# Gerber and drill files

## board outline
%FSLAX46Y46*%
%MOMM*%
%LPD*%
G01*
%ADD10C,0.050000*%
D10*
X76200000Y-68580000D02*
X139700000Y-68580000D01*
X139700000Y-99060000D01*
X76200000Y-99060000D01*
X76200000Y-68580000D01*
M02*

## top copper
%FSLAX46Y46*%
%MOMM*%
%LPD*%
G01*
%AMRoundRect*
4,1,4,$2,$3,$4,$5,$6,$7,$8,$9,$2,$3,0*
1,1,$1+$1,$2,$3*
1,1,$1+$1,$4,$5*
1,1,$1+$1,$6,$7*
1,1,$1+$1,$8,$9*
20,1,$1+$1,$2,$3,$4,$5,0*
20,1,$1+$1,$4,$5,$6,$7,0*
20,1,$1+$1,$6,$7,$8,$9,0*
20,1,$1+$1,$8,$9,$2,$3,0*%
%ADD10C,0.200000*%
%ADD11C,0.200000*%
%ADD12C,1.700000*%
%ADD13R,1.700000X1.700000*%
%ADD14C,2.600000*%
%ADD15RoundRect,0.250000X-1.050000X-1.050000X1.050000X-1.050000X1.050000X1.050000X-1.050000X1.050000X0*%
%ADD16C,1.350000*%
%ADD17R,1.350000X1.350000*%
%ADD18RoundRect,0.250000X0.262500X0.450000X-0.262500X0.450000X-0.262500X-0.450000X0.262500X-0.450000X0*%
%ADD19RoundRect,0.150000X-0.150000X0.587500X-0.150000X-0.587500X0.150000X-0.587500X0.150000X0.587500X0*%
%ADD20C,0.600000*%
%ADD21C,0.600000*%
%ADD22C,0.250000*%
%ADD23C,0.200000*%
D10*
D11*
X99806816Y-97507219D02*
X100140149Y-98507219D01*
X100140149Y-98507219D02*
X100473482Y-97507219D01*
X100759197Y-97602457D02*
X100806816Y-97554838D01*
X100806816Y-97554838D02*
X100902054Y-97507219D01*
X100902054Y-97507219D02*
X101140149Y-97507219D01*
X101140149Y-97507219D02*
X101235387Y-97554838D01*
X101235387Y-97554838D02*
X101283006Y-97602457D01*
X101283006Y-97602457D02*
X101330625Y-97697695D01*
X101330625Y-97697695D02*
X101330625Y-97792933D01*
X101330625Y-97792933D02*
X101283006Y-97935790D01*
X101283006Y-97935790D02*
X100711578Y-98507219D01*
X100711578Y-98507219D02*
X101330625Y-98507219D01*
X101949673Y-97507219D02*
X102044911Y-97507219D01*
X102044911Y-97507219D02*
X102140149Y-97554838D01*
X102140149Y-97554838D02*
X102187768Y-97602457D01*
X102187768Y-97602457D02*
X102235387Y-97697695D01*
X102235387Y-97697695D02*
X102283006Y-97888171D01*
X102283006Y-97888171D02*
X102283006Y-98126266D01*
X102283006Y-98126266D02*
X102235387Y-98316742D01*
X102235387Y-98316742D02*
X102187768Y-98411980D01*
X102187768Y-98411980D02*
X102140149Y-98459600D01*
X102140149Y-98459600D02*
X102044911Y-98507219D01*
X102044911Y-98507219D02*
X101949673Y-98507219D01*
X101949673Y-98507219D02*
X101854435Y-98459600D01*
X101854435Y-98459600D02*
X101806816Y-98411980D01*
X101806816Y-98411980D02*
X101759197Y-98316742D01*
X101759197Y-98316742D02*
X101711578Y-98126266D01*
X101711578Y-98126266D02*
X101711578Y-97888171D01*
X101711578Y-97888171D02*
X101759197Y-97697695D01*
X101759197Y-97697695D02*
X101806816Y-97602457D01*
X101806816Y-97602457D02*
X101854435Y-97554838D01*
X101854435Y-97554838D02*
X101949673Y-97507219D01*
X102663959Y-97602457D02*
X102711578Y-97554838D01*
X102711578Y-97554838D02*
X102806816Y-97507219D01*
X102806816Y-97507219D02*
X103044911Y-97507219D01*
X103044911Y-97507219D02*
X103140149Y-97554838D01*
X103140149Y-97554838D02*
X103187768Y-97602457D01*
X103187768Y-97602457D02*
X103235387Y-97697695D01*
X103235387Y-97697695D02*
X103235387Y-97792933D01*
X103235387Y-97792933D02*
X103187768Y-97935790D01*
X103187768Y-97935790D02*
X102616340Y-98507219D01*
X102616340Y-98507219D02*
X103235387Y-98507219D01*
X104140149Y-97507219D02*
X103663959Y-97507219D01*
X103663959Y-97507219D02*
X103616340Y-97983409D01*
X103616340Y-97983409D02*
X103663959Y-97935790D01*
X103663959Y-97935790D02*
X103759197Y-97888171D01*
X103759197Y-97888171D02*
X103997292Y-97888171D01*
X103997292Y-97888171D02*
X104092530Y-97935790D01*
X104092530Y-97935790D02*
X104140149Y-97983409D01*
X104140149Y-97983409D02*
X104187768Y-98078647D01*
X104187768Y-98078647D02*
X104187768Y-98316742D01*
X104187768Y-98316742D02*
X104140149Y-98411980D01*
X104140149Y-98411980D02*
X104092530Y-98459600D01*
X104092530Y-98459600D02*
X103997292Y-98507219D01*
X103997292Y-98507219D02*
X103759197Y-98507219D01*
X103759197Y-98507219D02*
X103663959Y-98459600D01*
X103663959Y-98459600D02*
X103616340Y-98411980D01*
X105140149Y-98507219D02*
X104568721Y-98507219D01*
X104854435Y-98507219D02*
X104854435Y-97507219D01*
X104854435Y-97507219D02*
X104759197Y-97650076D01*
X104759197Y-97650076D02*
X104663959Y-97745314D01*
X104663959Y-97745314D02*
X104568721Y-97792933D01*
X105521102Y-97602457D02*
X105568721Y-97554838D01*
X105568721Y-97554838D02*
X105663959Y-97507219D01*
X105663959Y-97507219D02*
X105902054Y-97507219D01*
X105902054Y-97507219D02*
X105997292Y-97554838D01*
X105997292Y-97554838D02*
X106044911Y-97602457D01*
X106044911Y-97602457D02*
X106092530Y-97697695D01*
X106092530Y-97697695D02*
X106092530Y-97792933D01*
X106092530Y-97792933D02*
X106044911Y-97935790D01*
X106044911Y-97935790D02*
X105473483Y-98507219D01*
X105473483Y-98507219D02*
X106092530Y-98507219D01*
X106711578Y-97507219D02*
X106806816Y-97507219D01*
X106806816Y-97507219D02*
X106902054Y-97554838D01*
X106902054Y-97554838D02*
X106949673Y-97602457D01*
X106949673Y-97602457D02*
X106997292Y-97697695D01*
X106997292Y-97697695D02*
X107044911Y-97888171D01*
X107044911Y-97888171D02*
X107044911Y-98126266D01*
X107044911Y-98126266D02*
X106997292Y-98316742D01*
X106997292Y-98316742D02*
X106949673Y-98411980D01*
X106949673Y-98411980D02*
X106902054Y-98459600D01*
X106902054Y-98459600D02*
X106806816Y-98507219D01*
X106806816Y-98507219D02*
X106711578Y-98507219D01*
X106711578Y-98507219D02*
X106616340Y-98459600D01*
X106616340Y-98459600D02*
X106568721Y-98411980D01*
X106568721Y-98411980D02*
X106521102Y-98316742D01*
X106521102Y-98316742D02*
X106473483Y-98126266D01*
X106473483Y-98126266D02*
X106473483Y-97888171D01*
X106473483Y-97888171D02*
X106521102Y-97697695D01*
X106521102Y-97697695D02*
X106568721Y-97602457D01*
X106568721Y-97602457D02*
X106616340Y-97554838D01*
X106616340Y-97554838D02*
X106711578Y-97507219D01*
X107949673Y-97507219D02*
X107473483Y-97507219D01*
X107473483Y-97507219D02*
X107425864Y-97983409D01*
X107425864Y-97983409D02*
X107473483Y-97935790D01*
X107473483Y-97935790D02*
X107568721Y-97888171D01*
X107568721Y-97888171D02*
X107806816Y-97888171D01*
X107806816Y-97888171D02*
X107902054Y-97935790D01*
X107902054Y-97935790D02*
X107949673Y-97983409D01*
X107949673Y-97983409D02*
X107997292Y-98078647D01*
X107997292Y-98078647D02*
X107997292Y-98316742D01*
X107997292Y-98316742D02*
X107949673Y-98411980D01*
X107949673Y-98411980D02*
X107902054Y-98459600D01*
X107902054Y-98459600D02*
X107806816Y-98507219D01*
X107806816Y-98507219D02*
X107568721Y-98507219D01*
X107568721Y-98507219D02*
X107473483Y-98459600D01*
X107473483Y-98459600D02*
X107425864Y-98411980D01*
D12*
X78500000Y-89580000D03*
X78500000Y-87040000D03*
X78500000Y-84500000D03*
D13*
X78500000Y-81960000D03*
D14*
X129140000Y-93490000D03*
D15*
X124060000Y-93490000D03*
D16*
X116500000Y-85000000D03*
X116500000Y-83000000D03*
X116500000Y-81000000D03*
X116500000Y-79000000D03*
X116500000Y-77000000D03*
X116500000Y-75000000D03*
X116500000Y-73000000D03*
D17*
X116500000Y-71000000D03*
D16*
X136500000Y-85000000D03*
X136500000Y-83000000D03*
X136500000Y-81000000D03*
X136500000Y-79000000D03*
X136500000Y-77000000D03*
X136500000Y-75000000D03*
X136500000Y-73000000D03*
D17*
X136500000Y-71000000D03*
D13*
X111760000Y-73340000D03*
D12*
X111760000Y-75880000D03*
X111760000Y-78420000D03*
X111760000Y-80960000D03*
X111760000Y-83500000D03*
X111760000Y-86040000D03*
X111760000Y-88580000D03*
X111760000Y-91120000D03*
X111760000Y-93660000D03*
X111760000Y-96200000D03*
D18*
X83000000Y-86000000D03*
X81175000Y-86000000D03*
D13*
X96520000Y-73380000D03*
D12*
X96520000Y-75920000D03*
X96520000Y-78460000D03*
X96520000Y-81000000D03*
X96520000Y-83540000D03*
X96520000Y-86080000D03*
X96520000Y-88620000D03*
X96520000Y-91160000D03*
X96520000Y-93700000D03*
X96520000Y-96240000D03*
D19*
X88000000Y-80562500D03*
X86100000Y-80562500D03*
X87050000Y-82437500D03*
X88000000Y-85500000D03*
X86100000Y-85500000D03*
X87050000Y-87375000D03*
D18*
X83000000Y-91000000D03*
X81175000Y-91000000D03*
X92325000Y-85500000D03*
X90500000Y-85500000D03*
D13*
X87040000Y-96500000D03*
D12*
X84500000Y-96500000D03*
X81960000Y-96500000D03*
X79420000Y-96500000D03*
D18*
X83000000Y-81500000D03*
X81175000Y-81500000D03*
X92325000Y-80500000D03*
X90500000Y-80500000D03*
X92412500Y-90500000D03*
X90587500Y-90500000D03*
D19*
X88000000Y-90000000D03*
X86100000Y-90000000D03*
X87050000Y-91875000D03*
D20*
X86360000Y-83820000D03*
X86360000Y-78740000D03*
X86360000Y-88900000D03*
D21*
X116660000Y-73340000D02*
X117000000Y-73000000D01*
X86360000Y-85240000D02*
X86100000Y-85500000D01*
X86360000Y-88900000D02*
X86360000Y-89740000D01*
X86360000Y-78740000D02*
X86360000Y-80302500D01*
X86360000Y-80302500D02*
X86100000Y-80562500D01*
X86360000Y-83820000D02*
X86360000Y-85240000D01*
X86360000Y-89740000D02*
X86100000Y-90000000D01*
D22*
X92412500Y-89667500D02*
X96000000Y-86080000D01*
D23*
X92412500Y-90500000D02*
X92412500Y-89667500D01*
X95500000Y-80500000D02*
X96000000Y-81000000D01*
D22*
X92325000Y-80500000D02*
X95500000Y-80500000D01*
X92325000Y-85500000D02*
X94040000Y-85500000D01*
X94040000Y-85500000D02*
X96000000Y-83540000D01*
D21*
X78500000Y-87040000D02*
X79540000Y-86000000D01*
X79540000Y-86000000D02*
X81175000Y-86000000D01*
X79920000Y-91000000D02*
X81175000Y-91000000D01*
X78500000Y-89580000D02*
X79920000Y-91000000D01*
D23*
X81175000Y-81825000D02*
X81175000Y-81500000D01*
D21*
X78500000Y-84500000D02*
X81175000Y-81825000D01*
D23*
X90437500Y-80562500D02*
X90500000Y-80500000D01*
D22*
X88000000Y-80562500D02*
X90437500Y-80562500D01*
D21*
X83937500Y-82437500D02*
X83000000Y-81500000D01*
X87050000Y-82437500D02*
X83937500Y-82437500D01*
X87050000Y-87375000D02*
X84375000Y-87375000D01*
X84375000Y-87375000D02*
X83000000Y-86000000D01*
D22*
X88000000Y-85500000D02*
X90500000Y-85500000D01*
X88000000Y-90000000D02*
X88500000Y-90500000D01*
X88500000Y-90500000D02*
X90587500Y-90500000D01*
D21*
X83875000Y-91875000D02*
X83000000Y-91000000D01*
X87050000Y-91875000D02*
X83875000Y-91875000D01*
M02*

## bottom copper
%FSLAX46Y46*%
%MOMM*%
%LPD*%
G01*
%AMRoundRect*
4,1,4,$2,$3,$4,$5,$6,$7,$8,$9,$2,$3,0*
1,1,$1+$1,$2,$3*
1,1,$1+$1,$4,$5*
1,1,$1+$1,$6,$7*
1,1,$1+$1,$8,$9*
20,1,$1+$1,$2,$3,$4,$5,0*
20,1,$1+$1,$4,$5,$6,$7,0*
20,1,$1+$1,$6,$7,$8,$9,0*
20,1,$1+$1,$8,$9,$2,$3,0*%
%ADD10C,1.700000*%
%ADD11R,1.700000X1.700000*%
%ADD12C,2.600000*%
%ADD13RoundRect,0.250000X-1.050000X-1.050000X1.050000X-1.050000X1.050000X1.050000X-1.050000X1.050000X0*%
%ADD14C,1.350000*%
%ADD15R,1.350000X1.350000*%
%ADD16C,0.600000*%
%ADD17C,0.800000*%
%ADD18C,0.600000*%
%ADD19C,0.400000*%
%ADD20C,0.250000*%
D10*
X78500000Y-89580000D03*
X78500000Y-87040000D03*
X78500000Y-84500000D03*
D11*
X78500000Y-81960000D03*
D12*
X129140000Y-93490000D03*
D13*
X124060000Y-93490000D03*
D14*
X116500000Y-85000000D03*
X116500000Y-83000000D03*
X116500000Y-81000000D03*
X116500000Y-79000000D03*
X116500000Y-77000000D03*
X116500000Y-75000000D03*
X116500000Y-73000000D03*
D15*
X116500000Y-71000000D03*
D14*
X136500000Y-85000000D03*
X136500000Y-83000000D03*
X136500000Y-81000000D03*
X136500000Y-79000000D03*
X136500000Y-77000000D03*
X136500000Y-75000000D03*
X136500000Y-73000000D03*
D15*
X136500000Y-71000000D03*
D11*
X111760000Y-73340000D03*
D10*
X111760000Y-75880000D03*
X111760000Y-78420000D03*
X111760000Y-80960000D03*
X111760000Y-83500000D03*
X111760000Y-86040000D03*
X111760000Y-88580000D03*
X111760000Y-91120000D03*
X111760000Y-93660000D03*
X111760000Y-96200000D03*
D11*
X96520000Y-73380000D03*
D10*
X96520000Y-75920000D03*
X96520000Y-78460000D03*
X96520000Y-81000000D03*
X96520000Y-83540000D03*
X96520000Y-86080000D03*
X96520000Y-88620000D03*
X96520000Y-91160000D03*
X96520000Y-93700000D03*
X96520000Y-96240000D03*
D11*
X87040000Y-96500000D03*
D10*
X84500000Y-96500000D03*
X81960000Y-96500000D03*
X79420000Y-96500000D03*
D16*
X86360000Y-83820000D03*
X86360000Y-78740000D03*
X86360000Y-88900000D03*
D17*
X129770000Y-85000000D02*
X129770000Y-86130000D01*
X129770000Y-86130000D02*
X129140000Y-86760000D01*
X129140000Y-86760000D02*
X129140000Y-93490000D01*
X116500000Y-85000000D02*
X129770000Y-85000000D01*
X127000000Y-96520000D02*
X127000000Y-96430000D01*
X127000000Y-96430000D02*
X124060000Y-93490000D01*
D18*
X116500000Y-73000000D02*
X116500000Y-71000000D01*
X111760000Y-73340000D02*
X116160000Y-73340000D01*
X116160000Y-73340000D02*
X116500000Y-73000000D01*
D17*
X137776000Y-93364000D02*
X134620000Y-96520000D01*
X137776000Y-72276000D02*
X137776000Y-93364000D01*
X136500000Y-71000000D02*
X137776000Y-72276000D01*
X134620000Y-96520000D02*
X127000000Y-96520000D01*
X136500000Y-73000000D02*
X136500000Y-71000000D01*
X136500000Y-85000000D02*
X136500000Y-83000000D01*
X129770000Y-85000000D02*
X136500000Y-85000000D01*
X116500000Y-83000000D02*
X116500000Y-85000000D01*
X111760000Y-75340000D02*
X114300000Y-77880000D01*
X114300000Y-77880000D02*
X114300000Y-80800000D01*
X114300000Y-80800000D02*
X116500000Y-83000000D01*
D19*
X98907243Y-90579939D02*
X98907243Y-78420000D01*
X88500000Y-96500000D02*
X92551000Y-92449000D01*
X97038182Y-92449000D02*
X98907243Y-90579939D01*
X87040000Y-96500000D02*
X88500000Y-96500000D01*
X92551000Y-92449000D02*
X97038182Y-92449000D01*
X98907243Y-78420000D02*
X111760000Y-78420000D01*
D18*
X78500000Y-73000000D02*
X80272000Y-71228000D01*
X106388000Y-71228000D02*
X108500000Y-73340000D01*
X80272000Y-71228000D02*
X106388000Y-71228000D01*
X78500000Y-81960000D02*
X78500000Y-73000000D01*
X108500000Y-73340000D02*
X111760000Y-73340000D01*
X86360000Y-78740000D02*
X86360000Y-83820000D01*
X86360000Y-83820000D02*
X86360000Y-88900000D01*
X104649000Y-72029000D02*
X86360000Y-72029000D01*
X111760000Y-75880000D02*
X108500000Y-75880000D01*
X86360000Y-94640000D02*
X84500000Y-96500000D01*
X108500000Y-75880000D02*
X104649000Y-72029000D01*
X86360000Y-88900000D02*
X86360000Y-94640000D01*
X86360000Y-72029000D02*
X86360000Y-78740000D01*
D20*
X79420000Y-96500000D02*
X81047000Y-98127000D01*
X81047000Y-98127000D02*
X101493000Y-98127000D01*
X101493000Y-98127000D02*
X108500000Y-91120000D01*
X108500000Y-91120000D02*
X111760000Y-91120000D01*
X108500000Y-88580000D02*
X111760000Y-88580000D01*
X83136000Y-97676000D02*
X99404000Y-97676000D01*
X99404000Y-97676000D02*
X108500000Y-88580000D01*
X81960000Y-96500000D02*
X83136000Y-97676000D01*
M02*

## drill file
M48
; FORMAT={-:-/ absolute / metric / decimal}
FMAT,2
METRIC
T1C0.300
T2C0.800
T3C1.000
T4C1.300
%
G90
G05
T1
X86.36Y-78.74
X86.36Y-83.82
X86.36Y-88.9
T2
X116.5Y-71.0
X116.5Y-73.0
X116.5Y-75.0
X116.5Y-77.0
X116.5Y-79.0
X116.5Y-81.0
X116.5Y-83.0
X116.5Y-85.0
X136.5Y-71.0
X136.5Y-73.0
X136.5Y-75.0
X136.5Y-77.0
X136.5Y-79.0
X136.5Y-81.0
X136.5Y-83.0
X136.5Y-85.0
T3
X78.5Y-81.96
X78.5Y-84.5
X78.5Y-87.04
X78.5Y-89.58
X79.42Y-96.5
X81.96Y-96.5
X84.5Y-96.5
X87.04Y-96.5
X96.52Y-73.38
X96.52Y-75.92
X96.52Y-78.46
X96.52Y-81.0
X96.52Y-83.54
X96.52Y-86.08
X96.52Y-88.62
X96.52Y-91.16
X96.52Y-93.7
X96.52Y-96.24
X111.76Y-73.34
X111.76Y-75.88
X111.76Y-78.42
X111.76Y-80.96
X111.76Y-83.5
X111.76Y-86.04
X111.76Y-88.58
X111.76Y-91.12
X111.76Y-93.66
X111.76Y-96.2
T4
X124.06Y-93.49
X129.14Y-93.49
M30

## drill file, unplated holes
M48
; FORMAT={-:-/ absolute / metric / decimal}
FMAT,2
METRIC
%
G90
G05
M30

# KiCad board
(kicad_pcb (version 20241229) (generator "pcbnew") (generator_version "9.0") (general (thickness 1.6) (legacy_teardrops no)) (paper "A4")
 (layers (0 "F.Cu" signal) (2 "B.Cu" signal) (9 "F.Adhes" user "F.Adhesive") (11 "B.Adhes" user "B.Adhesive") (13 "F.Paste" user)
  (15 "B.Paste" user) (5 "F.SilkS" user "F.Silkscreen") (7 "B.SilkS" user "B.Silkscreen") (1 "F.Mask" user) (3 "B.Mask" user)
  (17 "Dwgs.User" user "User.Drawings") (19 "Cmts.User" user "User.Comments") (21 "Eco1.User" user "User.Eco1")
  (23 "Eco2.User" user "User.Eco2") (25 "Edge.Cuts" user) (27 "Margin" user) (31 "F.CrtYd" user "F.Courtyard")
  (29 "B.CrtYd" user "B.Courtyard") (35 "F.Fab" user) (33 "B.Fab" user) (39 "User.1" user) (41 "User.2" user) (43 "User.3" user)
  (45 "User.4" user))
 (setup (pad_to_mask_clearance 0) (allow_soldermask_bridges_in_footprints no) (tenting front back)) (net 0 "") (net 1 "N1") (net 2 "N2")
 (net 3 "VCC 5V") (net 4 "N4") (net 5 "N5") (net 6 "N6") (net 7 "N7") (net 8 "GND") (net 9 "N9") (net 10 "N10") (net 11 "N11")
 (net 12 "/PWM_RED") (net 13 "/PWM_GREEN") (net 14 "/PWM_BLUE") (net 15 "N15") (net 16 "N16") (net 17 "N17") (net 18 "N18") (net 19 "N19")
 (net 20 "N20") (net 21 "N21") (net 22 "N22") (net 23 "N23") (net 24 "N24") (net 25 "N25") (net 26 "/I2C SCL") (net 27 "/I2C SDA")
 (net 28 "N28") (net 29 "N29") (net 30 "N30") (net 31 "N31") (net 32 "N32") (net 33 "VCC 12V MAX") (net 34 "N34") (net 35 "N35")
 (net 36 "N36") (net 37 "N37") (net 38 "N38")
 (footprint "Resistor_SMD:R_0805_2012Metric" (layer "F.Cu") (at 82.0875 86 180)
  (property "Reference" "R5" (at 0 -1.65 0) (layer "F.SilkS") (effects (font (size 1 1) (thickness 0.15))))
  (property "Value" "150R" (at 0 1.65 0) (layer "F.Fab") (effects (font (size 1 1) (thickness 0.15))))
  (pad "1" smd roundrect (at -0.9125 0 180) (size 1.025 1.4) (layers "F.Cu" "F.Mask" "F.Paste") (roundrect_rratio 0.243902) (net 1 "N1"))
  (pad "2" smd roundrect (at 0.9125 0 180) (size 1.025 1.4) (layers "F.Cu" "F.Mask" "F.Paste") (roundrect_rratio 0.243902) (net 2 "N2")))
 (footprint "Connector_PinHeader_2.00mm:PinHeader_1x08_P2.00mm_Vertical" (layer "F.Cu") (at 116.5 71)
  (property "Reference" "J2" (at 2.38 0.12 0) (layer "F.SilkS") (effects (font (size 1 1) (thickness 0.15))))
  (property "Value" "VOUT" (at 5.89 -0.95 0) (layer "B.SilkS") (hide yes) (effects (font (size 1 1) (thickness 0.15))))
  (pad "1" thru_hole rect (at 0 0) (size 1.35 1.35) (drill 0.8) (layers "*.Cu" "*.Mask") (remove_unused_layers no) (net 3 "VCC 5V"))
  (pad "2" thru_hole circle (at 0 2) (size 1.35 1.35) (drill 0.8) (layers "*.Cu" "*.Mask") (remove_unused_layers no) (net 3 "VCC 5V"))
  (pad "3" thru_hole circle (at 0 4) (size 1.35 1.35) (drill 0.8) (layers "*.Cu" "*.Mask") (remove_unused_layers no) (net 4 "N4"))
  (pad "4" thru_hole circle (at 0 6) (size 1.35 1.35) (drill 0.8) (layers "*.Cu" "*.Mask") (remove_unused_layers no) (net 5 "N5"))
  (pad "5" thru_hole circle (at 0 8) (size 1.35 1.35) (drill 0.8) (layers "*.Cu" "*.Mask") (remove_unused_layers no) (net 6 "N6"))
  (pad "6" thru_hole circle (at 0 10) (size 1.35 1.35) (drill 0.8) (layers "*.Cu" "*.Mask") (remove_unused_layers no) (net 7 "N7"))
  (pad "7" thru_hole circle (at 0 12) (size 1.35 1.35) (drill 0.8) (layers "*.Cu" "*.Mask") (remove_unused_layers no) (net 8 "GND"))
  (pad "8" thru_hole circle (at 0 14) (size 1.35 1.35) (drill 0.8) (layers "*.Cu" "*.Mask") (remove_unused_layers no) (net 8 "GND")))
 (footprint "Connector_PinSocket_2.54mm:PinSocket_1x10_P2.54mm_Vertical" (layer "F.Cu") (at 96.52 73.38)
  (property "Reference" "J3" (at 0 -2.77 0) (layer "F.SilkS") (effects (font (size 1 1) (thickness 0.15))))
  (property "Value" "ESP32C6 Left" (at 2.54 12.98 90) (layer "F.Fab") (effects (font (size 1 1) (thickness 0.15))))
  (pad "1" thru_hole rect (at 0 0) (size 1.7 1.7) (drill 1) (layers "*.Cu" "*.Mask") (remove_unused_layers no) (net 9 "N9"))
  (pad "2" thru_hole circle (at 0 2.54) (size 1.7 1.7) (drill 1) (layers "*.Cu" "*.Mask") (remove_unused_layers no) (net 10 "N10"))
  (pad "3" thru_hole circle (at 0 5.08) (size 1.7 1.7) (drill 1) (layers "*.Cu" "*.Mask") (remove_unused_layers no) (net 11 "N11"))
  (pad "4" thru_hole circle (at 0 7.62) (size 1.7 1.7) (drill 1) (layers "*.Cu" "*.Mask") (remove_unused_layers no) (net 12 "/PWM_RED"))
  (pad "5" thru_hole circle (at 0 10.16) (size 1.7 1.7) (drill 1) (layers "*.Cu" "*.Mask") (remove_unused_layers no) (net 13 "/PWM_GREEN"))
  (pad "6" thru_hole circle (at 0 12.7) (size 1.7 1.7) (drill 1) (layers "*.Cu" "*.Mask") (remove_unused_layers no) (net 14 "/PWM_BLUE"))
  (pad "7" thru_hole circle (at 0 15.24) (size 1.7 1.7) (drill 1) (layers "*.Cu" "*.Mask") (remove_unused_layers no) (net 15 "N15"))
  (pad "8" thru_hole circle (at 0 17.78) (size 1.7 1.7) (drill 1) (layers "*.Cu" "*.Mask") (remove_unused_layers no) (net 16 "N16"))
  (pad "9" thru_hole circle (at 0 20.32) (size 1.7 1.7) (drill 1) (layers "*.Cu" "*.Mask") (remove_unused_layers no) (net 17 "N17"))
  (pad "10" thru_hole circle (at 0 22.86) (size 1.7 1.7) (drill 1) (layers "*.Cu" "*.Mask") (remove_unused_layers no) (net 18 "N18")))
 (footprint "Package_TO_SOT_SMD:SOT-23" (layer "F.Cu") (at 87.05 81.5 -90)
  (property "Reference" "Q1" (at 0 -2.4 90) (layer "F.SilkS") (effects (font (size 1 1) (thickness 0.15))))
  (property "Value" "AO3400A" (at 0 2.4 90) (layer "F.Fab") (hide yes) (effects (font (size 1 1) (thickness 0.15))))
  (pad "1" smd roundrect (at -0.9375 -0.95 270) (size 1.475 0.6) (layers "F.Cu" "F.Mask" "F.Paste") (roundrect_rratio 0.25) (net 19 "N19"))
  (pad "2" smd roundrect (at -0.9375 0.95 270) (size 1.475 0.6) (layers "F.Cu" "F.Mask" "F.Paste") (roundrect_rratio 0.25) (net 8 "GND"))
  (pad "3" smd roundrect (at 0.9375 0 270) (size 1.475 0.6) (layers "F.Cu" "F.Mask" "F.Paste") (roundrect_rratio 0.25) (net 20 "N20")))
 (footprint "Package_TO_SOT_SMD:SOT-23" (layer "F.Cu") (at 87.05 86.4375 -90)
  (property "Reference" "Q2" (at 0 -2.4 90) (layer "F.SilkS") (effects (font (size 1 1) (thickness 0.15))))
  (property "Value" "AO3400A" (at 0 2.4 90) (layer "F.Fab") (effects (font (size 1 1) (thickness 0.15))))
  (pad "1" smd roundrect (at -0.9375 -0.95 270) (size 1.475 0.6) (layers "F.Cu" "F.Mask" "F.Paste") (roundrect_rratio 0.25) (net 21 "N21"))
  (pad "2" smd roundrect (at -0.9375 0.95 270) (size 1.475 0.6) (layers "F.Cu" "F.Mask" "F.Paste") (roundrect_rratio 0.25) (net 8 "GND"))
  (pad "3" smd roundrect (at 0.9375 0 270) (size 1.475 0.6) (layers "F.Cu" "F.Mask" "F.Paste") (roundrect_rratio 0.25) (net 1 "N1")))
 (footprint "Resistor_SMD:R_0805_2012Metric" (layer "F.Cu") (at 82.0875 91 180)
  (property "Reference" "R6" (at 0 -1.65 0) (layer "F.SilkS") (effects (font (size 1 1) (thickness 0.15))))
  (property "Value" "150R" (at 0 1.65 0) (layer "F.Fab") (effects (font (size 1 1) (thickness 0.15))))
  (pad "1" smd roundrect (at -0.9125 0 180) (size 1.025 1.4) (layers "F.Cu" "F.Mask" "F.Paste") (roundrect_rratio 0.243902) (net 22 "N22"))
  (pad "2" smd roundrect (at 0.9125 0 180) (size 1.025 1.4) (layers "F.Cu" "F.Mask" "F.Paste") (roundrect_rratio 0.243902) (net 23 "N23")))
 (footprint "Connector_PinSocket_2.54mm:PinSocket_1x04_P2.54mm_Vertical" (layer "F.Cu") (at 78.5 81.96)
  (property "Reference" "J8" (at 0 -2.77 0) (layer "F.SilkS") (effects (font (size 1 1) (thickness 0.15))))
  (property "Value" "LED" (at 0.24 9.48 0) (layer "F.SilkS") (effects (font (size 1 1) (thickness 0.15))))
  (pad "1" thru_hole rect (at 0 0) (size 1.7 1.7) (drill 1) (layers "*.Cu" "*.Mask") (remove_unused_layers no) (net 3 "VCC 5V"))
  (pad "2" thru_hole circle (at 0 2.54) (size 1.7 1.7) (drill 1) (layers "*.Cu" "*.Mask") (remove_unused_layers no) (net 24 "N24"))
  (pad "3" thru_hole circle (at 0 5.08) (size 1.7 1.7) (drill 1) (layers "*.Cu" "*.Mask") (remove_unused_layers no) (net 2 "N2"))
  (pad "4" thru_hole circle (at 0 7.62) (size 1.7 1.7) (drill 1) (layers "*.Cu" "*.Mask") (remove_unused_layers no) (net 23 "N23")))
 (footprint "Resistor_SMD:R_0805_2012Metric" (layer "F.Cu") (at 91.4125 85.5 180)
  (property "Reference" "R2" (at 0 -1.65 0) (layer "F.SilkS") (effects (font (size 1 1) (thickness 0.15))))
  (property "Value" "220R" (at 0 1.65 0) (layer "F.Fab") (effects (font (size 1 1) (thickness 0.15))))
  (pad "1" smd roundrect (at -0.9125 0 180) (size 1.025 1.4) (layers "F.Cu" "F.Mask" "F.Paste") (roundrect_rratio 0.243902)
   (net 13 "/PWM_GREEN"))
  (pad "2" smd roundrect (at 0.9125 0 180) (size 1.025 1.4) (layers "F.Cu" "F.Mask" "F.Paste") (roundrect_rratio 0.243902) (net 21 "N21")))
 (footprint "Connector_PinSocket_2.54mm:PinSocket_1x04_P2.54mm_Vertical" (layer "F.Cu") (at 87.04 96.5 -90)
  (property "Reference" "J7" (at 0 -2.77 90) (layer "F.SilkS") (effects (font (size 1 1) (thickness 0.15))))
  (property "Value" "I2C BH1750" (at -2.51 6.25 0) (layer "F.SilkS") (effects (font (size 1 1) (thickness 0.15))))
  (pad "1" thru_hole rect (at 0 0 270) (size 1.7 1.7) (drill 1) (layers "*.Cu" "*.Mask") (remove_unused_layers no) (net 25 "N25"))
  (pad "2" thru_hole circle (at 0 2.54 270) (size 1.7 1.7) (drill 1) (layers "*.Cu" "*.Mask") (remove_unused_layers no) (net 8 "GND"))
  (pad "3" thru_hole circle (at 0 5.08 270) (size 1.7 1.7) (drill 1) (layers "*.Cu" "*.Mask") (remove_unused_layers no) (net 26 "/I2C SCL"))
  (pad "4" thru_hole circle (at 0 7.62 270) (size 1.7 1.7) (drill 1) (layers "*.Cu" "*.Mask") (remove_unused_layers no) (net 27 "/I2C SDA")))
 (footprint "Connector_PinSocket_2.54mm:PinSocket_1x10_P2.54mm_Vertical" (layer "F.Cu") (at 111.76 73.34)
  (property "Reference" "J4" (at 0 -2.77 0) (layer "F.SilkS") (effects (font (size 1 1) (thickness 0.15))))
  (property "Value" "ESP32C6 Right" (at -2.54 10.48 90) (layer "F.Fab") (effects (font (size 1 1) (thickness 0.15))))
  (pad "1" thru_hole rect (at 0 0) (size 1.7 1.7) (drill 1) (layers "*.Cu" "*.Mask") (remove_unused_layers no) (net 3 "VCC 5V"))
  (pad "2" thru_hole circle (at 0 2.54) (size 1.7 1.7) (drill 1) (layers "*.Cu" "*.Mask") (remove_unused_layers no) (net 8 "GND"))
  (pad "3" thru_hole circle (at 0 5.08) (size 1.7 1.7) (drill 1) (layers "*.Cu" "*.Mask") (remove_unused_layers no) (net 25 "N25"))
  (pad "4" thru_hole circle (at 0 7.62) (size 1.7 1.7) (drill 1) (layers "*.Cu" "*.Mask") (remove_unused_layers no) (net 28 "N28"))
  (pad "5" thru_hole circle (at 0 10.16) (size 1.7 1.7) (drill 1) (layers "*.Cu" "*.Mask") (remove_unused_layers no) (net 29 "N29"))
  (pad "6" thru_hole circle (at 0 12.7) (size 1.7 1.7) (drill 1) (layers "*.Cu" "*.Mask") (remove_unused_layers no) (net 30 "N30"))
  (pad "7" thru_hole circle (at 0 15.24) (size 1.7 1.7) (drill 1) (layers "*.Cu" "*.Mask") (remove_unused_layers no) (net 26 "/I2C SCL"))
  (pad "8" thru_hole circle (at 0 17.78) (size 1.7 1.7) (drill 1) (layers "*.Cu" "*.Mask") (remove_unused_layers no) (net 27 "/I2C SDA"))
  (pad "9" thru_hole circle (at 0 20.32) (size 1.7 1.7) (drill 1) (layers "*.Cu" "*.Mask") (remove_unused_layers no) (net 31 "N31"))
  (pad "10" thru_hole circle (at 0 22.86) (size 1.7 1.7) (drill 1) (layers "*.Cu" "*.Mask") (remove_unused_layers no) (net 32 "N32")))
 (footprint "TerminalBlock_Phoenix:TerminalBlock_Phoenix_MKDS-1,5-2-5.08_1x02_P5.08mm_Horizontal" (layer "F.Cu") (at 124.06 93.49)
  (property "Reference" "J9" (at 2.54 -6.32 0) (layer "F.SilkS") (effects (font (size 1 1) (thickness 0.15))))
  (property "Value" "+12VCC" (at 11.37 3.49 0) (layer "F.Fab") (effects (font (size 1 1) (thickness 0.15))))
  (pad "1" thru_hole roundrect (at 0 0) (size 2.6 2.6) (drill 1.3) (layers "*.Cu" "*.Mask") (remove_unused_layers no)
   (roundrect_rratio 0.096154) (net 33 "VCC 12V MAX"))
  (pad "2" thru_hole circle (at 5.08 0) (size 2.6 2.6) (drill 1.3) (layers "*.Cu" "*.Mask") (remove_unused_layers no) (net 8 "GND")))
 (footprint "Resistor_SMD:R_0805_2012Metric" (layer "F.Cu") (at 82.0875 81.5 180)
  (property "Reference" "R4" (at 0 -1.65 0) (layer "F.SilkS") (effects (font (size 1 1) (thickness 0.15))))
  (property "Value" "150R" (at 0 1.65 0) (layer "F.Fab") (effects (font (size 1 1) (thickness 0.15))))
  (pad "1" smd roundrect (at -0.9125 0 180) (size 1.025 1.4) (layers "F.Cu" "F.Mask" "F.Paste") (roundrect_rratio 0.243902) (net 20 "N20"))
  (pad "2" smd roundrect (at 0.9125 0 180) (size 1.025 1.4) (layers "F.Cu" "F.Mask" "F.Paste") (roundrect_rratio 0.243902) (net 24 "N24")))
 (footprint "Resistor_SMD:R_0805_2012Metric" (layer "F.Cu") (at 91.4125 80.5 180)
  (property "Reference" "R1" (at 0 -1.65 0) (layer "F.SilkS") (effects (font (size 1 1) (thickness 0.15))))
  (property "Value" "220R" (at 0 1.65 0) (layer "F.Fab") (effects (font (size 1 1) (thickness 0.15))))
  (pad "1" smd roundrect (at -0.9125 0 180) (size 1.025 1.4) (layers "F.Cu" "F.Mask" "F.Paste") (roundrect_rratio 0.243902)
   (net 12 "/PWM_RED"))
  (pad "2" smd roundrect (at 0.9125 0 180) (size 1.025 1.4) (layers "F.Cu" "F.Mask" "F.Paste") (roundrect_rratio 0.243902) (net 19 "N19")))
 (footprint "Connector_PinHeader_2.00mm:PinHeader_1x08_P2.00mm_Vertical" (layer "F.Cu") (at 136.5 71)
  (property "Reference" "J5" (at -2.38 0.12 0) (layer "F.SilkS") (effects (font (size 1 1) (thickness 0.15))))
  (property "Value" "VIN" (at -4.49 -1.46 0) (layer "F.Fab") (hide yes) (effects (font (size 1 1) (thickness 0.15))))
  (pad "1" thru_hole rect (at 0 0) (size 1.35 1.35) (drill 0.8) (layers "*.Cu" "*.Mask") (remove_unused_layers no) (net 33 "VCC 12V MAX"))
  (pad "2" thru_hole circle (at 0 2) (size 1.35 1.35) (drill 0.8) (layers "*.Cu" "*.Mask") (remove_unused_layers no) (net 33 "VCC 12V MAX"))
  (pad "3" thru_hole circle (at 0 4) (size 1.35 1.35) (drill 0.8) (layers "*.Cu" "*.Mask") (remove_unused_layers no) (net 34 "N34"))
  (pad "4" thru_hole circle (at 0 6) (size 1.35 1.35) (drill 0.8) (layers "*.Cu" "*.Mask") (remove_unused_layers no) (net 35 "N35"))
  (pad "5" thru_hole circle (at 0 8) (size 1.35 1.35) (drill 0.8) (layers "*.Cu" "*.Mask") (remove_unused_layers no) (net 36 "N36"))
  (pad "6" thru_hole circle (at 0 10) (size 1.35 1.35) (drill 0.8) (layers "*.Cu" "*.Mask") (remove_unused_layers no) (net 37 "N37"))
  (pad "7" thru_hole circle (at 0 12) (size 1.35 1.35) (drill 0.8) (layers "*.Cu" "*.Mask") (remove_unused_layers no) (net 8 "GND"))
  (pad "8" thru_hole circle (at 0 14) (size 1.35 1.35) (drill 0.8) (layers "*.Cu" "*.Mask") (remove_unused_layers no) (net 8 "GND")))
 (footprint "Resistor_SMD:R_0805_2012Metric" (layer "F.Cu") (at 91.5 90.5 180)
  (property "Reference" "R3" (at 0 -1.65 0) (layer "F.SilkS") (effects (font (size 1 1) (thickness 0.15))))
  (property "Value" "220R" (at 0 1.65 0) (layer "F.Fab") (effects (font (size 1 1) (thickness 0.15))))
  (pad "1" smd roundrect (at -0.9125 0 180) (size 1.025 1.4) (layers "F.Cu" "F.Mask" "F.Paste") (roundrect_rratio 0.243902)
   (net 14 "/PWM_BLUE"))
  (pad "2" smd roundrect (at 0.9125 0 180) (size 1.025 1.4) (layers "F.Cu" "F.Mask" "F.Paste") (roundrect_rratio 0.243902) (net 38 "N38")))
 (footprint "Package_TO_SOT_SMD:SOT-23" (layer "F.Cu") (at 87.05 90.9375 -90)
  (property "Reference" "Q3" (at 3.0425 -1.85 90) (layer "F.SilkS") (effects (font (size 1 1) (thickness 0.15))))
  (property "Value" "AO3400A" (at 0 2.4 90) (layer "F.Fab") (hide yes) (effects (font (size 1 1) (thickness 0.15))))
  (pad "1" smd roundrect (at -0.9375 -0.95 270) (size 1.475 0.6) (layers "F.Cu" "F.Mask" "F.Paste") (roundrect_rratio 0.25) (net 38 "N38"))
  (pad "2" smd roundrect (at -0.9375 0.95 270) (size 1.475 0.6) (layers "F.Cu" "F.Mask" "F.Paste") (roundrect_rratio 0.25) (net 8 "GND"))
  (pad "3" smd roundrect (at 0.9375 0 270) (size 1.475 0.6) (layers "F.Cu" "F.Mask" "F.Paste") (roundrect_rratio 0.25) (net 22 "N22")))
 (gr_rect (start 76.2 68.58) (end 139.7 99.06) (stroke (width 0.05) (type default)) (fill no) (layer "Edge.Cuts"))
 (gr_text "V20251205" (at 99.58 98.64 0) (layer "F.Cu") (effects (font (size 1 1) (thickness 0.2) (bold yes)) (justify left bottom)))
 (segment (start 116.66 73.34) (end 117 73) (width 0.6) (layer "F.Cu") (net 3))
 (segment (start 78.5 73) (end 80.272 71.228) (width 0.6) (layer "B.Cu") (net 3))
 (segment (start 116.5 73) (end 116.5 71) (width 0.6) (layer "B.Cu") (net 3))
 (segment (start 106.388 71.228) (end 108.5 73.34) (width 0.6) (layer "B.Cu") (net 3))
 (segment (start 111.76 73.34) (end 116.16 73.34) (width 0.6) (layer "B.Cu") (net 3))
 (segment (start 116.16 73.34) (end 116.5 73) (width 0.6) (layer "B.Cu") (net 3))
 (segment (start 80.272 71.228) (end 106.388 71.228) (width 0.6) (layer "B.Cu") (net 3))
 (segment (start 78.5 81.96) (end 78.5 73) (width 0.6) (layer "B.Cu") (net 3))
 (segment (start 108.5 73.34) (end 111.76 73.34) (width 0.6) (layer "B.Cu") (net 3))
 (segment (start 86.36 85.24) (end 86.1 85.5) (width 0.6) (layer "F.Cu") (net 8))
 (segment (start 86.36 88.9) (end 86.36 89.74) (width 0.6) (layer "F.Cu") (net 8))
 (segment (start 86.36 78.74) (end 86.36 80.3025) (width 0.6) (layer "F.Cu") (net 8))
 (segment (start 86.36 80.3025) (end 86.1 80.5625) (width 0.6) (layer "F.Cu") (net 8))
 (segment (start 86.36 83.82) (end 86.36 85.24) (width 0.6) (layer "F.Cu") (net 8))
 (segment (start 86.36 89.74) (end 86.1 90) (width 0.6) (layer "F.Cu") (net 8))
 (via (at 86.36 83.82) (size 0.6) (drill 0.3) (layers "F.Cu" "B.Cu") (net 8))
 (via (at 86.36 78.74) (size 0.6) (drill 0.3) (layers "F.Cu" "B.Cu") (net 8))
 (via (at 86.36 88.9) (size 0.6) (drill 0.3) (layers "F.Cu" "B.Cu") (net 8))
 (segment (start 86.36 78.74) (end 86.36 83.82) (width 0.6) (layer "B.Cu") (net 8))
 (segment (start 136.5 85) (end 136.5 83) (width 0.8) (layer "B.Cu") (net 8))
 (segment (start 86.36 83.82) (end 86.36 88.9) (width 0.6) (layer "B.Cu") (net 8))
 (segment (start 129.14 86.76) (end 129.14 93.49) (width 0.8) (layer "B.Cu") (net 8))
 (segment (start 104.649 72.029) (end 86.36 72.029) (width 0.6) (layer "B.Cu") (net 8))
 (segment (start 111.76 75.34) (end 114.3 77.88) (width 0.8) (layer "B.Cu") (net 8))
 (segment (start 111.76 75.88) (end 108.5 75.88) (width 0.6) (layer "B.Cu") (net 8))
 (segment (start 129.77 86.13) (end 129.14 86.76) (width 0.8) (layer "B.Cu") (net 8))
 (segment (start 86.36 94.64) (end 84.5 96.5) (width 0.6) (layer "B.Cu") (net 8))
 (segment (start 129.77 85) (end 129.77 86.13) (width 0.8) (layer "B.Cu") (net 8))
 (segment (start 108.5 75.88) (end 104.649 72.029) (width 0.6) (layer "B.Cu") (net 8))
 (segment (start 114.3 77.88) (end 114.3 80.8) (width 0.8) (layer "B.Cu") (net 8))
 (segment (start 129.77 85) (end 136.5 85) (width 0.8) (layer "B.Cu") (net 8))
 (segment (start 86.36 88.9) (end 86.36 94.64) (width 0.6) (layer "B.Cu") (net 8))
 (segment (start 114.3 80.8) (end 116.5 83) (width 0.8) (layer "B.Cu") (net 8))
 (segment (start 86.36 72.029) (end 86.36 78.74) (width 0.6) (layer "B.Cu") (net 8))
 (segment (start 116.5 85) (end 129.77 85) (width 0.8) (layer "B.Cu") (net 8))
 (segment (start 116.5 83) (end 116.5 85) (width 0.8) (layer "B.Cu") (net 8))
 (segment (start 92.4125 89.6675) (end 96 86.08) (width 0.25) (layer "F.Cu") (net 14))
 (segment (start 92.4125 90.5) (end 92.4125 89.6675) (width 0.2) (layer "F.Cu") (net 14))
 (segment (start 95.5 80.5) (end 96 81) (width 0.2) (layer "F.Cu") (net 12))
 (segment (start 92.325 80.5) (end 95.5 80.5) (width 0.25) (layer "F.Cu") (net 12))
 (segment (start 92.325 85.5) (end 94.04 85.5) (width 0.25) (layer "F.Cu") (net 13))
 (segment (start 94.04 85.5) (end 96 83.54) (width 0.25) (layer "F.Cu") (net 13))
 (segment (start 79.42 96.5) (end 81.047 98.127) (width 0.25) (layer "B.Cu") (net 27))
 (segment (start 81.047 98.127) (end 101.493 98.127) (width 0.25) (layer "B.Cu") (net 27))
 (segment (start 101.493 98.127) (end 108.5 91.12) (width 0.25) (layer "B.Cu") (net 27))
 (segment (start 108.5 91.12) (end 111.76 91.12) (width 0.25) (layer "B.Cu") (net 27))
 (segment (start 108.5 88.58) (end 111.76 88.58) (width 0.25) (layer "B.Cu") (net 26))
 (segment (start 83.136 97.676) (end 99.404 97.676) (width 0.25) (layer "B.Cu") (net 26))
 (segment (start 99.404 97.676) (end 108.5 88.58) (width 0.25) (layer "B.Cu") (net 26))
 (segment (start 81.96 96.5) (end 83.136 97.676) (width 0.25) (layer "B.Cu") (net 26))
 (segment (start 92.551 92.449) (end 97.038182 92.449) (width 0.4) (layer "B.Cu") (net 25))
 (segment (start 97.038182 92.449) (end 98.907243 90.579939) (width 0.4) (layer "B.Cu") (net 25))
 (segment (start 88.5 96.5) (end 92.551 92.449) (width 0.4) (layer "B.Cu") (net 25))
 (segment (start 87.04 96.5) (end 88.5 96.5) (width 0.4) (layer "B.Cu") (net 25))
 (segment (start 98.907243 90.579939) (end 98.907243 78.42) (width 0.4) (layer "B.Cu") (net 25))
 (segment (start 98.907243 78.42) (end 111.76 78.42) (width 0.4) (layer "B.Cu") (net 25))
 (segment (start 137.776 72.276) (end 137.776 93.364) (width 0.8) (layer "B.Cu") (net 33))
 (segment (start 137.776 93.364) (end 134.62 96.52) (width 0.8) (layer "B.Cu") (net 33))
 (segment (start 127 96.52) (end 127 96.43) (width 0.8) (layer "B.Cu") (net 33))
 (segment (start 134.62 96.52) (end 127 96.52) (width 0.8) (layer "B.Cu") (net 33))
 (segment (start 136.5 71) (end 137.776 72.276) (width 0.8) (layer "B.Cu") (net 33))
 (segment (start 127 96.43) (end 124.06 93.49) (width 0.8) (layer "B.Cu") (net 33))
 (segment (start 136.5 73) (end 136.5 71) (width 0.8) (layer "B.Cu") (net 33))
 (segment (start 78.5 87.04) (end 79.54 86) (width 0.6) (layer "F.Cu") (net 2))
 (segment (start 79.54 86) (end 81.175 86) (width 0.6) (layer "F.Cu") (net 2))
 (segment (start 79.92 91) (end 81.175 91) (width 0.6) (layer "F.Cu") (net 23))
 (segment (start 78.5 89.58) (end 79.92 91) (width 0.6) (layer "F.Cu") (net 23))
 (segment (start 81.175 81.825) (end 81.175 81.5) (width 0.2) (layer "F.Cu") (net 24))
 (segment (start 78.5 84.5) (end 81.175 81.825) (width 0.6) (layer "F.Cu") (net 24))
 (segment (start 90.4375 80.5625) (end 90.5 80.5) (width 0.2) (layer "F.Cu") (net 19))
 (segment (start 88 80.5625) (end 90.4375 80.5625) (width 0.25) (layer "F.Cu") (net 19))
 (segment (start 83.9375 82.4375) (end 83 81.5) (width 0.6) (layer "F.Cu") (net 20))
 (segment (start 87.05 82.4375) (end 83.9375 82.4375) (width 0.6) (layer "F.Cu") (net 20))
 (segment (start 87.05 87.375) (end 84.375 87.375) (width 0.6) (layer "F.Cu") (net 1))
 (segment (start 84.375 87.375) (end 83 86) (width 0.6) (layer "F.Cu") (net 1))
 (segment (start 88 85.5) (end 90.5 85.5) (width 0.25) (layer "F.Cu") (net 21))
 (segment (start 88 90) (end 88.5 90.5) (width 0.25) (layer "F.Cu") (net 38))
 (segment (start 88.5 90.5) (end 90.5875 90.5) (width 0.25) (layer "F.Cu") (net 38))
 (segment (start 83.875 91.875) (end 83 91) (width 0.6) (layer "F.Cu") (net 22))
 (segment (start 87.05 91.875) (end 83.875 91.875) (width 0.6) (layer "F.Cu") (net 22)))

